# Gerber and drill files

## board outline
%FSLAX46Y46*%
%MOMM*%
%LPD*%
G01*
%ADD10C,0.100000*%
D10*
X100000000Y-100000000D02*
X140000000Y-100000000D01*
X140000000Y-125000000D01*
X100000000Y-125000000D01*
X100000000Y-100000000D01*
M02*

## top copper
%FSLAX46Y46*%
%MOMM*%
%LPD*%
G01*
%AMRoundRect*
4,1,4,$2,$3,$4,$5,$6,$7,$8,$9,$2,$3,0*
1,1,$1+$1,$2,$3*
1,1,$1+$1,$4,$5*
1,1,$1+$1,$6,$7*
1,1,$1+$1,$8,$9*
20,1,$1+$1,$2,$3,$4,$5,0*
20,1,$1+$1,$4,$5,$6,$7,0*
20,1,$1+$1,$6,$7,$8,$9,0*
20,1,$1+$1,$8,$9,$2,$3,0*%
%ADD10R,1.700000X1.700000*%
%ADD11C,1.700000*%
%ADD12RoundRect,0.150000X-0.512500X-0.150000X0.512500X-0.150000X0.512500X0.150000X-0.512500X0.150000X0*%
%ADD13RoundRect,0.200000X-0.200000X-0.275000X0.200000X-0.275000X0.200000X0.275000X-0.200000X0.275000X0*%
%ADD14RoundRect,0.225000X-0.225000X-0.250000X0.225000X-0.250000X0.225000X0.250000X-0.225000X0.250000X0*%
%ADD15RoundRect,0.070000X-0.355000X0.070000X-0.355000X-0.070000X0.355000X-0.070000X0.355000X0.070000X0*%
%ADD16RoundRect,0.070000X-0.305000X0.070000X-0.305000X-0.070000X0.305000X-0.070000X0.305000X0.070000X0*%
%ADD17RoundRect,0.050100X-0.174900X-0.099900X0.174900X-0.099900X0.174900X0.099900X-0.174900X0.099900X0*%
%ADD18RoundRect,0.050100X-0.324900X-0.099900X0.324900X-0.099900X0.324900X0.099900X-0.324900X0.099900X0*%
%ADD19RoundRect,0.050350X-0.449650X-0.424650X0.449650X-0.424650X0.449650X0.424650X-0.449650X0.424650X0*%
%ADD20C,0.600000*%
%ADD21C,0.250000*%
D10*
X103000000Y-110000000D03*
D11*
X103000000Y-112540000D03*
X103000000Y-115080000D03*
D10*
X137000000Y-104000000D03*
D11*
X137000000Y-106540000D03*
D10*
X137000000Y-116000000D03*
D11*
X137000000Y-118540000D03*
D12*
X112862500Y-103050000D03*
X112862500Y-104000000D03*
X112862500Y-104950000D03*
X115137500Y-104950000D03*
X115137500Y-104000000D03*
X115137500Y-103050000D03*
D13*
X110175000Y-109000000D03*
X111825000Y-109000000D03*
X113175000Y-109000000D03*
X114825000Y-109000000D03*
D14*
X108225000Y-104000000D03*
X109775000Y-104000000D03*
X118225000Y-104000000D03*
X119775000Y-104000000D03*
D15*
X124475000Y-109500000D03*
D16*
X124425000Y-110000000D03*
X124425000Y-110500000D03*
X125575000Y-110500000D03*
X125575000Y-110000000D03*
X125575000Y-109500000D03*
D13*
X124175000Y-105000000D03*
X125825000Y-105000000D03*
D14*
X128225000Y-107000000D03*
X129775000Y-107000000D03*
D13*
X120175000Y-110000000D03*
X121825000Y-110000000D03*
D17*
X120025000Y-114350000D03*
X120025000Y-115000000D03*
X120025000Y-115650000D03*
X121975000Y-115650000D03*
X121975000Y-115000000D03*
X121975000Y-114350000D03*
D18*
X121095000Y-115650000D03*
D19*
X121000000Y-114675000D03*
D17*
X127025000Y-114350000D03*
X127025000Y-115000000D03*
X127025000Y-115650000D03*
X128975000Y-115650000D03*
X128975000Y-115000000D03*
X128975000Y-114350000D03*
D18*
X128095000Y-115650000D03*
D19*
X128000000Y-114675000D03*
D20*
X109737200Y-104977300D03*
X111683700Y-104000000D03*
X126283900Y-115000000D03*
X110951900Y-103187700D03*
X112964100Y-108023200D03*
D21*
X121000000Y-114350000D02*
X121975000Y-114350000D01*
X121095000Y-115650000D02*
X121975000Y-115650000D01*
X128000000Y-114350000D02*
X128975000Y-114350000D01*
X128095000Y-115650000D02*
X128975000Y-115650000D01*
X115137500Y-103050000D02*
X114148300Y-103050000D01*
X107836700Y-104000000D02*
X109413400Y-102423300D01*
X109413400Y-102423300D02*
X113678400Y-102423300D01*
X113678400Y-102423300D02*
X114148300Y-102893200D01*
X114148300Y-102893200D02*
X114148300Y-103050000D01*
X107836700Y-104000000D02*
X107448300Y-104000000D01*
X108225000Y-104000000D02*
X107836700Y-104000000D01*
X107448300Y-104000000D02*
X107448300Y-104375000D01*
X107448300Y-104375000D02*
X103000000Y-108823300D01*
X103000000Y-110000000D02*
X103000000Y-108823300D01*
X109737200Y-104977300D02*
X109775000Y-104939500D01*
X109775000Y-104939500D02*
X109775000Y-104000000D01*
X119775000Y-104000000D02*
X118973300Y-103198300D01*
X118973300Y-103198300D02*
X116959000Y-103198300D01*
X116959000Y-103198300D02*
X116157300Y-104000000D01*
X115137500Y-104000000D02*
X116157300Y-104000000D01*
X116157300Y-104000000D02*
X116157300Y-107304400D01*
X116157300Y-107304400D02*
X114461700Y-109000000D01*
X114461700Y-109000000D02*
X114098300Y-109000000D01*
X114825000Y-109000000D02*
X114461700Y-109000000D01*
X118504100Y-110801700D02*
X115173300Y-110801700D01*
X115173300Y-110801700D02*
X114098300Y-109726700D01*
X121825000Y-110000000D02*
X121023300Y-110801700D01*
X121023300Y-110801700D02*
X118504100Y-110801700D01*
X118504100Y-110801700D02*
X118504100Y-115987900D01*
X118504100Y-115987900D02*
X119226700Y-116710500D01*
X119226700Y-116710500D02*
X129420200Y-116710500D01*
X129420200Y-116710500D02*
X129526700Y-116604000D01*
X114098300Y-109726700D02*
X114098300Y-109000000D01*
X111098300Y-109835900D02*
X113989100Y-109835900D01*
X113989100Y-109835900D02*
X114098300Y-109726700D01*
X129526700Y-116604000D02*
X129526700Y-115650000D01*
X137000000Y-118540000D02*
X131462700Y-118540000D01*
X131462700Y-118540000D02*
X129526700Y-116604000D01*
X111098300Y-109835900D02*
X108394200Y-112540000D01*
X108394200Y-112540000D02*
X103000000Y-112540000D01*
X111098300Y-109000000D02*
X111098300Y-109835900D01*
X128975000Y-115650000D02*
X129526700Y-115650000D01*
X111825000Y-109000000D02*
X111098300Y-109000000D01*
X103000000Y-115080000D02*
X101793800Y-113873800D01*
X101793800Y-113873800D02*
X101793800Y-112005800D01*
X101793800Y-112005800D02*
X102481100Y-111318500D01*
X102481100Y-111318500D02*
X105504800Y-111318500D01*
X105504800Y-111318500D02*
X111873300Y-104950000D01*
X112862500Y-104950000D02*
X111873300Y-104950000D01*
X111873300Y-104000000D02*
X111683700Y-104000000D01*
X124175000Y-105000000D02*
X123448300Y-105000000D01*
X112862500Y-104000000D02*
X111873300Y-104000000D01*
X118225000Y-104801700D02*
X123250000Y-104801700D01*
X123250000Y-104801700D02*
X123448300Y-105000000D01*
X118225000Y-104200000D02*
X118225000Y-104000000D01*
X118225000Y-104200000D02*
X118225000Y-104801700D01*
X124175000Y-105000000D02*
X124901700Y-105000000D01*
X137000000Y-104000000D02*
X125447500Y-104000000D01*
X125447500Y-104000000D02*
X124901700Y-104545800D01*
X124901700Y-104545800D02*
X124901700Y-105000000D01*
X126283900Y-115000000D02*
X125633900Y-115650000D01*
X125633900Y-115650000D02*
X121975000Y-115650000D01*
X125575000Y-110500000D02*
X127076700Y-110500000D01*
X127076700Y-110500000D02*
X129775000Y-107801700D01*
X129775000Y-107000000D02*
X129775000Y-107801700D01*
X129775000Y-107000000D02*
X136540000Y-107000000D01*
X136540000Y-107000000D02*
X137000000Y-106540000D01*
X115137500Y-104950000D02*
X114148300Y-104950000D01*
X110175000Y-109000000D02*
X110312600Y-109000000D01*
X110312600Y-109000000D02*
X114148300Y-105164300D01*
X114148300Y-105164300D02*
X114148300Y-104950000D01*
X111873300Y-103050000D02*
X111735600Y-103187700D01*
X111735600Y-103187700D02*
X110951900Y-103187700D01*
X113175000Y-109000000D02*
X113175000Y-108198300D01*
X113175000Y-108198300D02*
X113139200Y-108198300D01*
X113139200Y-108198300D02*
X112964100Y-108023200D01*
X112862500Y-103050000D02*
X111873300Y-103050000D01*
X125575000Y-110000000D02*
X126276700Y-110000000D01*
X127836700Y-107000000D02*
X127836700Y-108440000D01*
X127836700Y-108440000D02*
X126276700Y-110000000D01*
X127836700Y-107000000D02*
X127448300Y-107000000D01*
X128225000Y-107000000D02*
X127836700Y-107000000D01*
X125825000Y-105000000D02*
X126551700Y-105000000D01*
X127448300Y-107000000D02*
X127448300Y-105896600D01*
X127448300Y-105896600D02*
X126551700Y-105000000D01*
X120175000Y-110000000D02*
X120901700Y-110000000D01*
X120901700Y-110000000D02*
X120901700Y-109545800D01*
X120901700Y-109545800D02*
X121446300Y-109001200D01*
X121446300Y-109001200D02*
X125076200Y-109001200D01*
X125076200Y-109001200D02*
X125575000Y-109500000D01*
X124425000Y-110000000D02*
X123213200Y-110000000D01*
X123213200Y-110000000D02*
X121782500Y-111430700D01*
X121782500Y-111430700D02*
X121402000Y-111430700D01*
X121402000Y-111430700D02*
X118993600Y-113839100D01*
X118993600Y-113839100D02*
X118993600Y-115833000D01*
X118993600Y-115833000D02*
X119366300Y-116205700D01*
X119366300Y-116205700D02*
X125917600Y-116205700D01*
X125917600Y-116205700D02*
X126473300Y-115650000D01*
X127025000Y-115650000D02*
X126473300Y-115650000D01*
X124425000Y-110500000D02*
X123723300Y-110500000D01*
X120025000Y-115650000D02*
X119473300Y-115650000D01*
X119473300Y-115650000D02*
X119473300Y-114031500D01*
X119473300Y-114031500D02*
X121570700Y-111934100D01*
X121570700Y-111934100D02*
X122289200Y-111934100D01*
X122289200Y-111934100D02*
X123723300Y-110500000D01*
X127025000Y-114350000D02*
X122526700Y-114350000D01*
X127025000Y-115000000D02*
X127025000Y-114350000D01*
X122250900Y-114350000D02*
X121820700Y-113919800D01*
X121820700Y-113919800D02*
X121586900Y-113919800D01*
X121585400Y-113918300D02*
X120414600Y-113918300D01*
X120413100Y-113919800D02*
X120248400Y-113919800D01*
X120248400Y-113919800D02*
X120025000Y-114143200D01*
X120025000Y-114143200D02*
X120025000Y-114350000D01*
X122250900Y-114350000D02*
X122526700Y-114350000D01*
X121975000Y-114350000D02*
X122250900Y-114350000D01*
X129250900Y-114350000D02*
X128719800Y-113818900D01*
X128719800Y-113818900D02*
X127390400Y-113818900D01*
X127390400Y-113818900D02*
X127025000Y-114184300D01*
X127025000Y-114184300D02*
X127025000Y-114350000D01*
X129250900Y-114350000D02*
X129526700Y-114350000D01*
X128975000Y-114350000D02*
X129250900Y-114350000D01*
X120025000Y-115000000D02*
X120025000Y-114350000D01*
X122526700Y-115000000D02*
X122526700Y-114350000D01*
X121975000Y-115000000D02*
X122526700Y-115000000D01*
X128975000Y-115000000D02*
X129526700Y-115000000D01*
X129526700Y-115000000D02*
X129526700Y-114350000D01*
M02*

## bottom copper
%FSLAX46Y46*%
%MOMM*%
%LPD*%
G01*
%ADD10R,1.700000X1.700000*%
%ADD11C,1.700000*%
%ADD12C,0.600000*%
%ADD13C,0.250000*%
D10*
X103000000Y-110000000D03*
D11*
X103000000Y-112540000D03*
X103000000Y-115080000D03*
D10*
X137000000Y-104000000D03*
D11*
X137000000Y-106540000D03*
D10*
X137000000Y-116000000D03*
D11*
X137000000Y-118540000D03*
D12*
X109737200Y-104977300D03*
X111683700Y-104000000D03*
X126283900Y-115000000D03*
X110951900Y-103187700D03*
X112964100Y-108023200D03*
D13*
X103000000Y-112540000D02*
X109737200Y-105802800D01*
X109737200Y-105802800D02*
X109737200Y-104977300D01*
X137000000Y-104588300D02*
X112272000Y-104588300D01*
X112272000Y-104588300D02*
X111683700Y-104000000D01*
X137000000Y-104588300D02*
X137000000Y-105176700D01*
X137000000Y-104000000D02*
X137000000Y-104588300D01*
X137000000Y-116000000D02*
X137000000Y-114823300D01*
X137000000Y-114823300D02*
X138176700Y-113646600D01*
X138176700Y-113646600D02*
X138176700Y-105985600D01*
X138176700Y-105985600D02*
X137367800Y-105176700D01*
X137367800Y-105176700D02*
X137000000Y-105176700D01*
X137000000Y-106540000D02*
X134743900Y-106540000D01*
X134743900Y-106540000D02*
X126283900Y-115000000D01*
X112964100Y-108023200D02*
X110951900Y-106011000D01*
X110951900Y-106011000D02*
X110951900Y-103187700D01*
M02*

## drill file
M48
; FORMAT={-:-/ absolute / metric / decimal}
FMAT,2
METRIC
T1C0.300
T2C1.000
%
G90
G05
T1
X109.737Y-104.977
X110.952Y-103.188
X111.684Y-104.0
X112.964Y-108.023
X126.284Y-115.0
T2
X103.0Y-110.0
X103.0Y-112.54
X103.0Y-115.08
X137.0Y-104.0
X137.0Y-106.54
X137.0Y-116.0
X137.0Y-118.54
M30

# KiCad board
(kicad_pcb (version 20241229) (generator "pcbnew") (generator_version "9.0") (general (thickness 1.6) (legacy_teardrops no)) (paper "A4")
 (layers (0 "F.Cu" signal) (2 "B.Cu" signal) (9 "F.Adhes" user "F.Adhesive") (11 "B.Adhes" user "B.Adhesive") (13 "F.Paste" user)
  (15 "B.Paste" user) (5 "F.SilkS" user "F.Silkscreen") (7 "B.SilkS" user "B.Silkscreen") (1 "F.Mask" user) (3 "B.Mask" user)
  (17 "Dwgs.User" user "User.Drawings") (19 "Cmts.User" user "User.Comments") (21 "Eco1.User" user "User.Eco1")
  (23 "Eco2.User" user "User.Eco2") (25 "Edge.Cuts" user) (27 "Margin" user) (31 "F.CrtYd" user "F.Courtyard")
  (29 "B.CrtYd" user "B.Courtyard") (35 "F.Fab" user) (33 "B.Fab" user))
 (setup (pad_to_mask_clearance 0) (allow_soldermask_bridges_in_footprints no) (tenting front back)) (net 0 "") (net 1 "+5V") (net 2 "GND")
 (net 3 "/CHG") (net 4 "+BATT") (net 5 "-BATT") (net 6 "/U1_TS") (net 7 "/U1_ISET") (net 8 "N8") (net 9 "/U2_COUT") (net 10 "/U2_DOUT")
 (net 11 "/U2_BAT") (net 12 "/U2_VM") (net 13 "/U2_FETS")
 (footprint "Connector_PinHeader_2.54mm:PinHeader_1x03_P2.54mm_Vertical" (layer "F.Cu") (at 103 110)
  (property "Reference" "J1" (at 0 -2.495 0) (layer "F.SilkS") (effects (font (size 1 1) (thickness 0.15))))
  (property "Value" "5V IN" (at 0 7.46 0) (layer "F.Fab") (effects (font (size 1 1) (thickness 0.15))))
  (pad "1" thru_hole rect (at 0 0) (size 1.7 1.7) (drill 1) (layers "*.Cu" "*.Mask") (remove_unused_layers no) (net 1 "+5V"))
  (pad "2" thru_hole circle (at 0 2.54) (size 1.7 1.7) (drill 1) (layers "*.Cu" "*.Mask") (remove_unused_layers no) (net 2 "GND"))
  (pad "3" thru_hole circle (at 0 5.08) (size 1.7 1.7) (drill 1) (layers "*.Cu" "*.Mask") (remove_unused_layers no) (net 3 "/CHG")))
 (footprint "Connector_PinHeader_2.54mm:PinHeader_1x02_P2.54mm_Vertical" (layer "F.Cu") (at 137 104)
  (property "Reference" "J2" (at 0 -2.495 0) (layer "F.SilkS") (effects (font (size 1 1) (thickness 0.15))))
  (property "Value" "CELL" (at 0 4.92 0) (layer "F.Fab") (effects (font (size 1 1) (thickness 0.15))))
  (pad "1" thru_hole rect (at 0 0) (size 1.7 1.7) (drill 1) (layers "*.Cu" "*.Mask") (remove_unused_layers no) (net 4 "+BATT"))
  (pad "2" thru_hole circle (at 0 2.54) (size 1.7 1.7) (drill 1) (layers "*.Cu" "*.Mask") (remove_unused_layers no) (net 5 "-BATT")))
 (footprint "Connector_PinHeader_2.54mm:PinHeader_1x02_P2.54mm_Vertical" (layer "F.Cu") (at 137 116)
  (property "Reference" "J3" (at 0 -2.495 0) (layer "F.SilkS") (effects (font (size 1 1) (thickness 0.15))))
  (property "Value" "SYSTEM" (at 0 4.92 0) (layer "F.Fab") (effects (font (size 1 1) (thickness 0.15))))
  (pad "1" thru_hole rect (at 0 0) (size 1.7 1.7) (drill 1) (layers "*.Cu" "*.Mask") (remove_unused_layers no) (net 4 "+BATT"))
  (pad "2" thru_hole circle (at 0 2.54) (size 1.7 1.7) (drill 1) (layers "*.Cu" "*.Mask") (remove_unused_layers no) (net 2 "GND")))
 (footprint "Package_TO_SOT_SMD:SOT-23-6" (layer "F.Cu") (at 114 104)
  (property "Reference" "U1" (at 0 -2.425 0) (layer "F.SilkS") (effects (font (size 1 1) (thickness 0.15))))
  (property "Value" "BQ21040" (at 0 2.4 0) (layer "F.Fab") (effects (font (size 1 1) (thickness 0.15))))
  (pad "1" smd roundrect (at -1.1375 -0.95) (size 1.325 0.6) (layers "F.Cu" "F.Mask" "F.Paste") (roundrect_rratio 0.25) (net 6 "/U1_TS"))
  (pad "2" smd roundrect (at -1.1375 0) (size 1.325 0.6) (layers "F.Cu" "F.Mask" "F.Paste") (roundrect_rratio 0.25) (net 4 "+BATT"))
  (pad "3" smd roundrect (at -1.1375 0.95) (size 1.325 0.6) (layers "F.Cu" "F.Mask" "F.Paste") (roundrect_rratio 0.25) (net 3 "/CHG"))
  (pad "4" smd roundrect (at 1.1375 0.95) (size 1.325 0.6) (layers "F.Cu" "F.Mask" "F.Paste") (roundrect_rratio 0.25) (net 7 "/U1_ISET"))
  (pad "5" smd roundrect (at 1.1375 0) (size 1.325 0.6) (layers "F.Cu" "F.Mask" "F.Paste") (roundrect_rratio 0.25) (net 2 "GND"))
  (pad "6" smd roundrect (at 1.1375 -0.95) (size 1.325 0.6) (layers "F.Cu" "F.Mask" "F.Paste") (roundrect_rratio 0.25) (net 1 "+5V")))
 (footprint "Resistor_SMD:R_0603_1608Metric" (layer "F.Cu") (at 111 109)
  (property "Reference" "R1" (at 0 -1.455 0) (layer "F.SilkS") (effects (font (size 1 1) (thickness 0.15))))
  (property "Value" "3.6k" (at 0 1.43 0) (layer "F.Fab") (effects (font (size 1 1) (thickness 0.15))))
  (pad "1" smd roundrect (at -0.825 0) (size 0.8 0.95) (layers "F.Cu" "F.Mask" "F.Paste") (roundrect_rratio 0.25) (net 7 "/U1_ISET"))
  (pad "2" smd roundrect (at 0.825 0) (size 0.8 0.95) (layers "F.Cu" "F.Mask" "F.Paste") (roundrect_rratio 0.25) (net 2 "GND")))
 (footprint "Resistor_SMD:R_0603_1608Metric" (layer "F.Cu") (at 114 109)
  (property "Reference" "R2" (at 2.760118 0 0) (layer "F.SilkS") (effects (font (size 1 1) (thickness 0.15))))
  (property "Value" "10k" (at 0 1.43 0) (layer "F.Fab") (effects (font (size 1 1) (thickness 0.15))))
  (pad "1" smd roundrect (at -0.825 0) (size 0.8 0.95) (layers "F.Cu" "F.Mask" "F.Paste") (roundrect_rratio 0.25) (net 6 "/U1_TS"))
  (pad "2" smd roundrect (at 0.825 0) (size 0.8 0.95) (layers "F.Cu" "F.Mask" "F.Paste") (roundrect_rratio 0.25) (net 2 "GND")))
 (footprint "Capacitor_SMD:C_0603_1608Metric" (layer "F.Cu") (at 109 104)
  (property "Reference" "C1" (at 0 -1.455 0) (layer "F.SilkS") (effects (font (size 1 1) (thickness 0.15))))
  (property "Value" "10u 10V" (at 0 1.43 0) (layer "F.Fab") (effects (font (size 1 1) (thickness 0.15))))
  (pad "1" smd roundrect (at -0.775 0) (size 0.9 0.95) (layers "F.Cu" "F.Mask" "F.Paste") (roundrect_rratio 0.25) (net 1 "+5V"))
  (pad "2" smd roundrect (at 0.775 0) (size 0.9 0.95) (layers "F.Cu" "F.Mask" "F.Paste") (roundrect_rratio 0.25) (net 2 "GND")))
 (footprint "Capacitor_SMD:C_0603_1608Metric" (layer "F.Cu") (at 119 104)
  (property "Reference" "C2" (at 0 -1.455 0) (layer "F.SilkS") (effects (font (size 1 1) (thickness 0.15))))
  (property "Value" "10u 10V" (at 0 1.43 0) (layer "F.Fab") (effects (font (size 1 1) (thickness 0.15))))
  (pad "1" smd roundrect (at -0.775 0) (size 0.9 0.95) (layers "F.Cu" "F.Mask" "F.Paste") (roundrect_rratio 0.25) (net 4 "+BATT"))
  (pad "2" smd roundrect (at 0.775 0) (size 0.9 0.95) (layers "F.Cu" "F.Mask" "F.Paste") (roundrect_rratio 0.25) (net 2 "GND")))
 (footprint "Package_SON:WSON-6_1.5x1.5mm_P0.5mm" (layer "F.Cu") (at 125 110)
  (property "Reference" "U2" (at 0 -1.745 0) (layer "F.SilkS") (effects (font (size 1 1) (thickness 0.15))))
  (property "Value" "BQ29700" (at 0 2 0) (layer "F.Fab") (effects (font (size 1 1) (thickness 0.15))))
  (pad "1" smd roundrect (at -0.525 -0.5 270) (size 0.28 0.85) (layers "F.Cu" "F.Mask" "F.Paste") (roundrect_rratio 0.25) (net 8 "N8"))
  (pad "2" smd roundrect (at -0.575 0 270) (size 0.28 0.75) (layers "F.Cu" "F.Mask" "F.Paste") (roundrect_rratio 0.25) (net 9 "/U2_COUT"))
  (pad "3" smd roundrect (at -0.575 0.5 270) (size 0.28 0.75) (layers "F.Cu" "F.Mask" "F.Paste") (roundrect_rratio 0.25) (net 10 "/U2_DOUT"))
  (pad "4" smd roundrect (at 0.575 0.5 270) (size 0.28 0.75) (layers "F.Cu" "F.Mask" "F.Paste") (roundrect_rratio 0.25) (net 5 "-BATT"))
  (pad "5" smd roundrect (at 0.575 0 270) (size 0.28 0.75) (layers "F.Cu" "F.Mask" "F.Paste") (roundrect_rratio 0.25) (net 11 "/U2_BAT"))
  (pad "6" smd roundrect (at 0.575 -0.5 270) (size 0.28 0.75) (layers "F.Cu" "F.Mask" "F.Paste") (roundrect_rratio 0.25) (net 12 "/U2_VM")))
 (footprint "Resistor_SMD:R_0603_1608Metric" (layer "F.Cu") (at 125 105)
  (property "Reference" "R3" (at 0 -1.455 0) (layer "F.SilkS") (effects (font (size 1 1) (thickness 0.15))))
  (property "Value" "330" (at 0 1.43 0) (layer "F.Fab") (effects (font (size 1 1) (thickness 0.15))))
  (pad "1" smd roundrect (at -0.825 0) (size 0.8 0.95) (layers "F.Cu" "F.Mask" "F.Paste") (roundrect_rratio 0.25) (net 4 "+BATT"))
  (pad "2" smd roundrect (at 0.825 0) (size 0.8 0.95) (layers "F.Cu" "F.Mask" "F.Paste") (roundrect_rratio 0.25) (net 11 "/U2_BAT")))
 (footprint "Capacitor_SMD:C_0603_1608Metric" (layer "F.Cu") (at 129 107)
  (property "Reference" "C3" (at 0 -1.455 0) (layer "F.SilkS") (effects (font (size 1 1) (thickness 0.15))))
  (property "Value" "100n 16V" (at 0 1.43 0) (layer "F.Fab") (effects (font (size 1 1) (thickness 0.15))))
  (pad "1" smd roundrect (at -0.775 0) (size 0.9 0.95) (layers "F.Cu" "F.Mask" "F.Paste") (roundrect_rratio 0.25) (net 11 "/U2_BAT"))
  (pad "2" smd roundrect (at 0.775 0) (size 0.9 0.95) (layers "F.Cu" "F.Mask" "F.Paste") (roundrect_rratio 0.25) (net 5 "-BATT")))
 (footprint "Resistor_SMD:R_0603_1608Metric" (layer "F.Cu") (at 121 110)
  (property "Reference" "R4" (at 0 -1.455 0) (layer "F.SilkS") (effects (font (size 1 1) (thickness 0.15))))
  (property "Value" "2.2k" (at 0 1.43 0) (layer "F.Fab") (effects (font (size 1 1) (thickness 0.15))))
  (pad "1" smd roundrect (at -0.825 0) (size 0.8 0.95) (layers "F.Cu" "F.Mask" "F.Paste") (roundrect_rratio 0.25) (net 12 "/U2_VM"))
  (pad "2" smd roundrect (at 0.825 0) (size 0.8 0.95) (layers "F.Cu" "F.Mask" "F.Paste") (roundrect_rratio 0.25) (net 2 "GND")))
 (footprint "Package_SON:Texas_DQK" (layer "F.Cu") (at 121 115)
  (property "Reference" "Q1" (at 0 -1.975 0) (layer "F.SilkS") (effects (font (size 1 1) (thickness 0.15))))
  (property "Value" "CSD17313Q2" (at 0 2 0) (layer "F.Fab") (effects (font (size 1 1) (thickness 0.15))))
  (pad "" smd roundrect (at 0 -0.325) (size 0.9 0.86) (layers "F.Paste") (roundrect_rratio 0.058))
  (pad "" smd roundrect (at 0.095 0.65) (size 0.7 0.29) (layers "F.Paste") (roundrect_rratio 0.172))
  (pad "1" smd roundrect (at -0.975 -0.65) (size 0.45 0.3) (layers "F.Cu" "F.Mask" "F.Paste") (roundrect_rratio 0.167) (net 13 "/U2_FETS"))
  (pad "2" smd roundrect (at -0.975 0) (size 0.45 0.3) (layers "F.Cu" "F.Mask" "F.Paste") (roundrect_rratio 0.167) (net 13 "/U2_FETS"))
  (pad "3" smd roundrect (at -0.975 0.65) (size 0.45 0.3) (layers "F.Cu" "F.Mask" "F.Paste") (roundrect_rratio 0.167) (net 10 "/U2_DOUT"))
  (pad "4" smd roundrect (at 0.975 0.65) (size 0.45 0.3) (layers "F.Cu" "F.Mask" "F.Paste") (roundrect_rratio 0.167) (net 5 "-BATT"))
  (pad "5" smd roundrect (at 0.975 0) (size 0.45 0.3) (layers "F.Cu" "F.Mask" "F.Paste") (roundrect_rratio 0.167) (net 13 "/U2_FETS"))
  (pad "6" smd roundrect (at 0.975 -0.65) (size 0.45 0.3) (layers "F.Cu" "F.Mask" "F.Paste") (roundrect_rratio 0.167) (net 13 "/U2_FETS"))
  (pad "7" smd roundrect (at 0.095 0.65) (size 0.75 0.3) (layers "F.Cu" "F.Mask") (roundrect_rratio 0.167) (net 5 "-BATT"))
  (pad "8" smd roundrect (at 0 -0.325) (size 1 0.95) (layers "F.Cu" "F.Mask") (roundrect_rratio 0.053) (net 13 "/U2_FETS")))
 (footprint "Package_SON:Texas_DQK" (layer "F.Cu") (at 128 115)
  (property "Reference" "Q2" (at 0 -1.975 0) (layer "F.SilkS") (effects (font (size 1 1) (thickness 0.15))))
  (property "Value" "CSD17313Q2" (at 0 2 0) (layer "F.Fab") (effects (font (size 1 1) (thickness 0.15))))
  (pad "" smd roundrect (at 0 -0.325) (size 0.9 0.86) (layers "F.Paste") (roundrect_rratio 0.058))
  (pad "" smd roundrect (at 0.095 0.65) (size 0.7 0.29) (layers "F.Paste") (roundrect_rratio 0.172))
  (pad "1" smd roundrect (at -0.975 -0.65) (size 0.45 0.3) (layers "F.Cu" "F.Mask" "F.Paste") (roundrect_rratio 0.167) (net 13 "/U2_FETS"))
  (pad "2" smd roundrect (at -0.975 0) (size 0.45 0.3) (layers "F.Cu" "F.Mask" "F.Paste") (roundrect_rratio 0.167) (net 13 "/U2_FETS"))
  (pad "3" smd roundrect (at -0.975 0.65) (size 0.45 0.3) (layers "F.Cu" "F.Mask" "F.Paste") (roundrect_rratio 0.167) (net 9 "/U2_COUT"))
  (pad "4" smd roundrect (at 0.975 0.65) (size 0.45 0.3) (layers "F.Cu" "F.Mask" "F.Paste") (roundrect_rratio 0.167) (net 2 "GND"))
  (pad "5" smd roundrect (at 0.975 0) (size 0.45 0.3) (layers "F.Cu" "F.Mask" "F.Paste") (roundrect_rratio 0.167) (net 13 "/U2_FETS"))
  (pad "6" smd roundrect (at 0.975 -0.65) (size 0.45 0.3) (layers "F.Cu" "F.Mask" "F.Paste") (roundrect_rratio 0.167) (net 13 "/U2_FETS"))
  (pad "7" smd roundrect (at 0.095 0.65) (size 0.75 0.3) (layers "F.Cu" "F.Mask") (roundrect_rratio 0.167) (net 2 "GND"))
  (pad "8" smd roundrect (at 0 -0.325) (size 1 0.95) (layers "F.Cu" "F.Mask") (roundrect_rratio 0.053) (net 13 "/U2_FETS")))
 (gr_rect (start 100 100) (end 140 125) (stroke (width 0.1) (type default)) (fill no) (layer "Edge.Cuts"))
 (segment (start 121 114.35) (end 121.975 114.35) (width 0.25) (layer "F.Cu") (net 13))
 (segment (start 121.095 115.65) (end 121.975 115.65) (width 0.25) (layer "F.Cu") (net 5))
 (segment (start 128 114.35) (end 128.975 114.35) (width 0.25) (layer "F.Cu") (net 13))
 (segment (start 128.095 115.65) (end 128.975 115.65) (width 0.25) (layer "F.Cu") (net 2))
 (segment (start 115.1375 103.05) (end 114.1483 103.05) (width 0.25) (layer "F.Cu") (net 1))
 (segment (start 107.8367 104) (end 109.4134 102.4233) (width 0.25) (layer "F.Cu") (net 1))
 (segment (start 109.4134 102.4233) (end 113.6784 102.4233) (width 0.25) (layer "F.Cu") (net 1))
 (segment (start 113.6784 102.4233) (end 114.1483 102.8932) (width 0.25) (layer "F.Cu") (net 1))
 (segment (start 114.1483 102.8932) (end 114.1483 103.05) (width 0.25) (layer "F.Cu") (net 1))
 (segment (start 107.8367 104) (end 107.4483 104) (width 0.25) (layer "F.Cu") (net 1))
 (segment (start 108.225 104) (end 107.8367 104) (width 0.25) (layer "F.Cu") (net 1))
 (segment (start 107.4483 104) (end 107.4483 104.375) (width 0.25) (layer "F.Cu") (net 1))
 (segment (start 107.4483 104.375) (end 103 108.8233) (width 0.25) (layer "F.Cu") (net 1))
 (segment (start 103 110) (end 103 108.8233) (width 0.25) (layer "F.Cu") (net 1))
 (segment (start 109.7372 104.9773) (end 109.775 104.9395) (width 0.25) (layer "F.Cu") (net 2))
 (segment (start 109.775 104.9395) (end 109.775 104) (width 0.25) (layer "F.Cu") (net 2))
 (segment (start 103 112.54) (end 109.7372 105.8028) (width 0.25) (layer "B.Cu") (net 2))
 (segment (start 109.7372 105.8028) (end 109.7372 104.9773) (width 0.25) (layer "B.Cu") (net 2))
 (segment (start 119.775 104) (end 118.9733 103.1983) (width 0.25) (layer "F.Cu") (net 2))
 (segment (start 118.9733 103.1983) (end 116.959 103.1983) (width 0.25) (layer "F.Cu") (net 2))
 (segment (start 116.959 103.1983) (end 116.1573 104) (width 0.25) (layer "F.Cu") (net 2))
 (segment (start 115.1375 104) (end 116.1573 104) (width 0.25) (layer "F.Cu") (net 2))
 (segment (start 116.1573 104) (end 116.1573 107.3044) (width 0.25) (layer "F.Cu") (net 2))
 (segment (start 116.1573 107.3044) (end 114.4617 109) (width 0.25) (layer "F.Cu") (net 2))
 (segment (start 114.4617 109) (end 114.0983 109) (width 0.25) (layer "F.Cu") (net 2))
 (segment (start 114.825 109) (end 114.4617 109) (width 0.25) (layer "F.Cu") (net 2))
 (segment (start 118.5041 110.8017) (end 115.1733 110.8017) (width 0.25) (layer "F.Cu") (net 2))
 (segment (start 115.1733 110.8017) (end 114.0983 109.7267) (width 0.25) (layer "F.Cu") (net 2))
 (segment (start 121.825 110) (end 121.0233 110.8017) (width 0.25) (layer "F.Cu") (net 2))
 (segment (start 121.0233 110.8017) (end 118.5041 110.8017) (width 0.25) (layer "F.Cu") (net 2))
 (segment (start 118.5041 110.8017) (end 118.5041 115.9879) (width 0.25) (layer "F.Cu") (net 2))
 (segment (start 118.5041 115.9879) (end 119.2267 116.7105) (width 0.25) (layer "F.Cu") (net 2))
 (segment (start 119.2267 116.7105) (end 129.4202 116.7105) (width 0.25) (layer "F.Cu") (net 2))
 (segment (start 129.4202 116.7105) (end 129.5267 116.604) (width 0.25) (layer "F.Cu") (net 2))
 (segment (start 114.0983 109.7267) (end 114.0983 109) (width 0.25) (layer "F.Cu") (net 2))
 (segment (start 111.0983 109.8359) (end 113.9891 109.8359) (width 0.25) (layer "F.Cu") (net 2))
 (segment (start 113.9891 109.8359) (end 114.0983 109.7267) (width 0.25) (layer "F.Cu") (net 2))
 (segment (start 129.5267 116.604) (end 129.5267 115.65) (width 0.25) (layer "F.Cu") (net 2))
 (segment (start 137 118.54) (end 131.4627 118.54) (width 0.25) (layer "F.Cu") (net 2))
 (segment (start 131.4627 118.54) (end 129.5267 116.604) (width 0.25) (layer "F.Cu") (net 2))
 (segment (start 111.0983 109.8359) (end 108.3942 112.54) (width 0.25) (layer "F.Cu") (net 2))
 (segment (start 108.3942 112.54) (end 103 112.54) (width 0.25) (layer "F.Cu") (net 2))
 (segment (start 111.0983 109) (end 111.0983 109.8359) (width 0.25) (layer "F.Cu") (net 2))
 (segment (start 128.975 115.65) (end 129.5267 115.65) (width 0.25) (layer "F.Cu") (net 2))
 (segment (start 111.825 109) (end 111.0983 109) (width 0.25) (layer "F.Cu") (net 2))
 (segment (start 103 115.08) (end 101.7938 113.8738) (width 0.25) (layer "F.Cu") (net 3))
 (segment (start 101.7938 113.8738) (end 101.7938 112.0058) (width 0.25) (layer "F.Cu") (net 3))
 (segment (start 101.7938 112.0058) (end 102.4811 111.3185) (width 0.25) (layer "F.Cu") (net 3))
 (segment (start 102.4811 111.3185) (end 105.5048 111.3185) (width 0.25) (layer "F.Cu") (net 3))
 (segment (start 105.5048 111.3185) (end 111.8733 104.95) (width 0.25) (layer "F.Cu") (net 3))
 (segment (start 112.8625 104.95) (end 111.8733 104.95) (width 0.25) (layer "F.Cu") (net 3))
 (segment (start 111.8733 104) (end 111.6837 104) (width 0.25) (layer "F.Cu") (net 4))
 (segment (start 137 104.5883) (end 112.272 104.5883) (width 0.25) (layer "B.Cu") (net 4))
 (segment (start 112.272 104.5883) (end 111.6837 104) (width 0.25) (layer "B.Cu") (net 4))
 (segment (start 124.175 105) (end 123.4483 105) (width 0.25) (layer "F.Cu") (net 4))
 (segment (start 112.8625 104) (end 111.8733 104) (width 0.25) (layer "F.Cu") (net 4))
 (segment (start 137 104.5883) (end 137 105.1767) (width 0.25) (layer "B.Cu") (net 4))
 (segment (start 137 104) (end 137 104.5883) (width 0.25) (layer "B.Cu") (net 4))
 (segment (start 118.225 104.8017) (end 123.25 104.8017) (width 0.25) (layer "F.Cu") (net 4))
 (segment (start 123.25 104.8017) (end 123.4483 105) (width 0.25) (layer "F.Cu") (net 4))
 (segment (start 118.225 104.2) (end 118.225 104) (width 0.25) (layer "F.Cu") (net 4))
 (segment (start 118.225 104.2) (end 118.225 104.8017) (width 0.25) (layer "F.Cu") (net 4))
 (segment (start 124.175 105) (end 124.9017 105) (width 0.25) (layer "F.Cu") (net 4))
 (segment (start 137 104) (end 125.4475 104) (width 0.25) (layer "F.Cu") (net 4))
 (segment (start 125.4475 104) (end 124.9017 104.5458) (width 0.25) (layer "F.Cu") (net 4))
 (segment (start 124.9017 104.5458) (end 124.9017 105) (width 0.25) (layer "F.Cu") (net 4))
 (segment (start 137 116) (end 137 114.8233) (width 0.25) (layer "B.Cu") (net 4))
 (segment (start 137 114.8233) (end 138.1767 113.6466) (width 0.25) (layer "B.Cu") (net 4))
 (segment (start 138.1767 113.6466) (end 138.1767 105.9856) (width 0.25) (layer "B.Cu") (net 4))
 (segment (start 138.1767 105.9856) (end 137.3678 105.1767) (width 0.25) (layer "B.Cu") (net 4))
 (segment (start 137.3678 105.1767) (end 137 105.1767) (width 0.25) (layer "B.Cu") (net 4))
 (segment (start 126.2839 115) (end 125.6339 115.65) (width 0.25) (layer "F.Cu") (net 5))
 (segment (start 125.6339 115.65) (end 121.975 115.65) (width 0.25) (layer "F.Cu") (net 5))
 (segment (start 137 106.54) (end 134.7439 106.54) (width 0.25) (layer "B.Cu") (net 5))
 (segment (start 134.7439 106.54) (end 126.2839 115) (width 0.25) (layer "B.Cu") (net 5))
 (segment (start 125.575 110.5) (end 127.0767 110.5) (width 0.25) (layer "F.Cu") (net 5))
 (segment (start 127.0767 110.5) (end 129.775 107.8017) (width 0.25) (layer "F.Cu") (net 5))
 (segment (start 129.775 107) (end 129.775 107.8017) (width 0.25) (layer "F.Cu") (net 5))
 (segment (start 129.775 107) (end 136.54 107) (width 0.25) (layer "F.Cu") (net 5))
 (segment (start 136.54 107) (end 137 106.54) (width 0.25) (layer "F.Cu") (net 5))
 (segment (start 115.1375 104.95) (end 114.1483 104.95) (width 0.25) (layer "F.Cu") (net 7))
 (segment (start 110.175 109) (end 110.3126 109) (width 0.25) (layer "F.Cu") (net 7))
 (segment (start 110.3126 109) (end 114.1483 105.1643) (width 0.25) (layer "F.Cu") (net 7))
 (segment (start 114.1483 105.1643) (end 114.1483 104.95) (width 0.25) (layer "F.Cu") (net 7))
 (segment (start 111.8733 103.05) (end 111.7356 103.1877) (width 0.25) (layer "F.Cu") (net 6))
 (segment (start 111.7356 103.1877) (end 110.9519 103.1877) (width 0.25) (layer "F.Cu") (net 6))
 (segment (start 112.9641 108.0232) (end 110.9519 106.011) (width 0.25) (layer "B.Cu") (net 6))
 (segment (start 110.9519 106.011) (end 110.9519 103.1877) (width 0.25) (layer "B.Cu") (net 6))
 (segment (start 113.175 109) (end 113.175 108.1983) (width 0.25) (layer "F.Cu") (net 6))
 (segment (start 113.175 108.1983) (end 113.1392 108.1983) (width 0.25) (layer "F.Cu") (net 6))
 (segment (start 113.1392 108.1983) (end 112.9641 108.0232) (width 0.25) (layer "F.Cu") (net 6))
 (segment (start 112.8625 103.05) (end 111.8733 103.05) (width 0.25) (layer "F.Cu") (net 6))
 (segment (start 125.575 110) (end 126.2767 110) (width 0.25) (layer "F.Cu") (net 11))
 (segment (start 127.8367 107) (end 127.8367 108.44) (width 0.25) (layer "F.Cu") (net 11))
 (segment (start 127.8367 108.44) (end 126.2767 110) (width 0.25) (layer "F.Cu") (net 11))
 (segment (start 127.8367 107) (end 127.4483 107) (width 0.25) (layer "F.Cu") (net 11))
 (segment (start 128.225 107) (end 127.8367 107) (width 0.25) (layer "F.Cu") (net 11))
 (segment (start 125.825 105) (end 126.5517 105) (width 0.25) (layer "F.Cu") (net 11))
 (segment (start 127.4483 107) (end 127.4483 105.8966) (width 0.25) (layer "F.Cu") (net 11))
 (segment (start 127.4483 105.8966) (end 126.5517 105) (width 0.25) (layer "F.Cu") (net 11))
 (segment (start 120.175 110) (end 120.9017 110) (width 0.25) (layer "F.Cu") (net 12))
 (segment (start 120.9017 110) (end 120.9017 109.5458) (width 0.25) (layer "F.Cu") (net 12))
 (segment (start 120.9017 109.5458) (end 121.4463 109.0012) (width 0.25) (layer "F.Cu") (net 12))
 (segment (start 121.4463 109.0012) (end 125.0762 109.0012) (width 0.25) (layer "F.Cu") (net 12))
 (segment (start 125.0762 109.0012) (end 125.575 109.5) (width 0.25) (layer "F.Cu") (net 12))
 (segment (start 124.425 110) (end 123.2132 110) (width 0.25) (layer "F.Cu") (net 9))
 (segment (start 123.2132 110) (end 121.7825 111.4307) (width 0.25) (layer "F.Cu") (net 9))
 (segment (start 121.7825 111.4307) (end 121.402 111.4307) (width 0.25) (layer "F.Cu") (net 9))
 (segment (start 121.402 111.4307) (end 118.9936 113.8391) (width 0.25) (layer "F.Cu") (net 9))
 (segment (start 118.9936 113.8391) (end 118.9936 115.833) (width 0.25) (layer "F.Cu") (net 9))
 (segment (start 118.9936 115.833) (end 119.3663 116.2057) (width 0.25) (layer "F.Cu") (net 9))
 (segment (start 119.3663 116.2057) (end 125.9176 116.2057) (width 0.25) (layer "F.Cu") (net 9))
 (segment (start 125.9176 116.2057) (end 126.4733 115.65) (width 0.25) (layer "F.Cu") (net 9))
 (segment (start 127.025 115.65) (end 126.4733 115.65) (width 0.25) (layer "F.Cu") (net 9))
 (segment (start 124.425 110.5) (end 123.7233 110.5) (width 0.25) (layer "F.Cu") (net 10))
 (segment (start 120.025 115.65) (end 119.4733 115.65) (width 0.25) (layer "F.Cu") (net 10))
 (segment (start 119.4733 115.65) (end 119.4733 114.0315) (width 0.25) (layer "F.Cu") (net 10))
 (segment (start 119.4733 114.0315) (end 121.5707 111.9341) (width 0.25) (layer "F.Cu") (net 10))
 (segment (start 121.5707 111.9341) (end 122.2892 111.9341) (width 0.25) (layer "F.Cu") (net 10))
 (segment (start 122.2892 111.9341) (end 123.7233 110.5) (width 0.25) (layer "F.Cu") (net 10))
 (segment (start 127.025 114.35) (end 122.5267 114.35) (width 0.25) (layer "F.Cu") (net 13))
 (segment (start 127.025 115) (end 127.025 114.35) (width 0.25) (layer "F.Cu") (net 13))
 (segment (start 122.2509 114.35) (end 121.8207 113.9198) (width 0.25) (layer "F.Cu") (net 13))
 (segment (start 121.8207 113.9198) (end 121.5869 113.9198) (width 0.25) (layer "F.Cu") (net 13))
 (segment (start 121.5854 113.9183) (end 120.4146 113.9183) (width 0.25) (layer "F.Cu") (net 13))
 (segment (start 120.4131 113.9198) (end 120.2484 113.9198) (width 0.25) (layer "F.Cu") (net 13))
 (segment (start 120.2484 113.9198) (end 120.025 114.1432) (width 0.25) (layer "F.Cu") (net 13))
 (segment (start 120.025 114.1432) (end 120.025 114.35) (width 0.25) (layer "F.Cu") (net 13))
 (segment (start 122.2509 114.35) (end 122.5267 114.35) (width 0.25) (layer "F.Cu") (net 13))
 (segment (start 121.975 114.35) (end 122.2509 114.35) (width 0.25) (layer "F.Cu") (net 13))
 (segment (start 129.2509 114.35) (end 128.7198 113.8189) (width 0.25) (layer "F.Cu") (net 13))
 (segment (start 128.7198 113.8189) (end 127.3904 113.8189) (width 0.25) (layer "F.Cu") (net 13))
 (segment (start 127.3904 113.8189) (end 127.025 114.1843) (width 0.25) (layer "F.Cu") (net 13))
 (segment (start 127.025 114.1843) (end 127.025 114.35) (width 0.25) (layer "F.Cu") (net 13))
 (segment (start 129.2509 114.35) (end 129.5267 114.35) (width 0.25) (layer "F.Cu") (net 13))
 (segment (start 128.975 114.35) (end 129.2509 114.35) (width 0.25) (layer "F.Cu") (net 13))
 (segment (start 120.025 115) (end 120.025 114.35) (width 0.25) (layer "F.Cu") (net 13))
 (segment (start 122.5267 115) (end 122.5267 114.35) (width 0.25) (layer "F.Cu") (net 13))
 (segment (start 121.975 115) (end 122.5267 115) (width 0.25) (layer "F.Cu") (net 13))
 (segment (start 128.975 115) (end 129.5267 115) (width 0.25) (layer "F.Cu") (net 13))
 (segment (start 129.5267 115) (end 129.5267 114.35) (width 0.25) (layer "F.Cu") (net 13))
 (via (at 109.7372 104.9773) (size 0.6) (drill 0.3) (layers "F.Cu" "B.Cu") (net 2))
 (via (at 111.6837 104) (size 0.6) (drill 0.3) (layers "F.Cu" "B.Cu") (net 4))
 (via (at 126.2839 115) (size 0.6) (drill 0.3) (layers "F.Cu" "B.Cu") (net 5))
 (via (at 110.9519 103.1877) (size 0.6) (drill 0.3) (layers "F.Cu" "B.Cu") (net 6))
 (via (at 112.9641 108.0232) (size 0.6) (drill 0.3) (layers "F.Cu" "B.Cu") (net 6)))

